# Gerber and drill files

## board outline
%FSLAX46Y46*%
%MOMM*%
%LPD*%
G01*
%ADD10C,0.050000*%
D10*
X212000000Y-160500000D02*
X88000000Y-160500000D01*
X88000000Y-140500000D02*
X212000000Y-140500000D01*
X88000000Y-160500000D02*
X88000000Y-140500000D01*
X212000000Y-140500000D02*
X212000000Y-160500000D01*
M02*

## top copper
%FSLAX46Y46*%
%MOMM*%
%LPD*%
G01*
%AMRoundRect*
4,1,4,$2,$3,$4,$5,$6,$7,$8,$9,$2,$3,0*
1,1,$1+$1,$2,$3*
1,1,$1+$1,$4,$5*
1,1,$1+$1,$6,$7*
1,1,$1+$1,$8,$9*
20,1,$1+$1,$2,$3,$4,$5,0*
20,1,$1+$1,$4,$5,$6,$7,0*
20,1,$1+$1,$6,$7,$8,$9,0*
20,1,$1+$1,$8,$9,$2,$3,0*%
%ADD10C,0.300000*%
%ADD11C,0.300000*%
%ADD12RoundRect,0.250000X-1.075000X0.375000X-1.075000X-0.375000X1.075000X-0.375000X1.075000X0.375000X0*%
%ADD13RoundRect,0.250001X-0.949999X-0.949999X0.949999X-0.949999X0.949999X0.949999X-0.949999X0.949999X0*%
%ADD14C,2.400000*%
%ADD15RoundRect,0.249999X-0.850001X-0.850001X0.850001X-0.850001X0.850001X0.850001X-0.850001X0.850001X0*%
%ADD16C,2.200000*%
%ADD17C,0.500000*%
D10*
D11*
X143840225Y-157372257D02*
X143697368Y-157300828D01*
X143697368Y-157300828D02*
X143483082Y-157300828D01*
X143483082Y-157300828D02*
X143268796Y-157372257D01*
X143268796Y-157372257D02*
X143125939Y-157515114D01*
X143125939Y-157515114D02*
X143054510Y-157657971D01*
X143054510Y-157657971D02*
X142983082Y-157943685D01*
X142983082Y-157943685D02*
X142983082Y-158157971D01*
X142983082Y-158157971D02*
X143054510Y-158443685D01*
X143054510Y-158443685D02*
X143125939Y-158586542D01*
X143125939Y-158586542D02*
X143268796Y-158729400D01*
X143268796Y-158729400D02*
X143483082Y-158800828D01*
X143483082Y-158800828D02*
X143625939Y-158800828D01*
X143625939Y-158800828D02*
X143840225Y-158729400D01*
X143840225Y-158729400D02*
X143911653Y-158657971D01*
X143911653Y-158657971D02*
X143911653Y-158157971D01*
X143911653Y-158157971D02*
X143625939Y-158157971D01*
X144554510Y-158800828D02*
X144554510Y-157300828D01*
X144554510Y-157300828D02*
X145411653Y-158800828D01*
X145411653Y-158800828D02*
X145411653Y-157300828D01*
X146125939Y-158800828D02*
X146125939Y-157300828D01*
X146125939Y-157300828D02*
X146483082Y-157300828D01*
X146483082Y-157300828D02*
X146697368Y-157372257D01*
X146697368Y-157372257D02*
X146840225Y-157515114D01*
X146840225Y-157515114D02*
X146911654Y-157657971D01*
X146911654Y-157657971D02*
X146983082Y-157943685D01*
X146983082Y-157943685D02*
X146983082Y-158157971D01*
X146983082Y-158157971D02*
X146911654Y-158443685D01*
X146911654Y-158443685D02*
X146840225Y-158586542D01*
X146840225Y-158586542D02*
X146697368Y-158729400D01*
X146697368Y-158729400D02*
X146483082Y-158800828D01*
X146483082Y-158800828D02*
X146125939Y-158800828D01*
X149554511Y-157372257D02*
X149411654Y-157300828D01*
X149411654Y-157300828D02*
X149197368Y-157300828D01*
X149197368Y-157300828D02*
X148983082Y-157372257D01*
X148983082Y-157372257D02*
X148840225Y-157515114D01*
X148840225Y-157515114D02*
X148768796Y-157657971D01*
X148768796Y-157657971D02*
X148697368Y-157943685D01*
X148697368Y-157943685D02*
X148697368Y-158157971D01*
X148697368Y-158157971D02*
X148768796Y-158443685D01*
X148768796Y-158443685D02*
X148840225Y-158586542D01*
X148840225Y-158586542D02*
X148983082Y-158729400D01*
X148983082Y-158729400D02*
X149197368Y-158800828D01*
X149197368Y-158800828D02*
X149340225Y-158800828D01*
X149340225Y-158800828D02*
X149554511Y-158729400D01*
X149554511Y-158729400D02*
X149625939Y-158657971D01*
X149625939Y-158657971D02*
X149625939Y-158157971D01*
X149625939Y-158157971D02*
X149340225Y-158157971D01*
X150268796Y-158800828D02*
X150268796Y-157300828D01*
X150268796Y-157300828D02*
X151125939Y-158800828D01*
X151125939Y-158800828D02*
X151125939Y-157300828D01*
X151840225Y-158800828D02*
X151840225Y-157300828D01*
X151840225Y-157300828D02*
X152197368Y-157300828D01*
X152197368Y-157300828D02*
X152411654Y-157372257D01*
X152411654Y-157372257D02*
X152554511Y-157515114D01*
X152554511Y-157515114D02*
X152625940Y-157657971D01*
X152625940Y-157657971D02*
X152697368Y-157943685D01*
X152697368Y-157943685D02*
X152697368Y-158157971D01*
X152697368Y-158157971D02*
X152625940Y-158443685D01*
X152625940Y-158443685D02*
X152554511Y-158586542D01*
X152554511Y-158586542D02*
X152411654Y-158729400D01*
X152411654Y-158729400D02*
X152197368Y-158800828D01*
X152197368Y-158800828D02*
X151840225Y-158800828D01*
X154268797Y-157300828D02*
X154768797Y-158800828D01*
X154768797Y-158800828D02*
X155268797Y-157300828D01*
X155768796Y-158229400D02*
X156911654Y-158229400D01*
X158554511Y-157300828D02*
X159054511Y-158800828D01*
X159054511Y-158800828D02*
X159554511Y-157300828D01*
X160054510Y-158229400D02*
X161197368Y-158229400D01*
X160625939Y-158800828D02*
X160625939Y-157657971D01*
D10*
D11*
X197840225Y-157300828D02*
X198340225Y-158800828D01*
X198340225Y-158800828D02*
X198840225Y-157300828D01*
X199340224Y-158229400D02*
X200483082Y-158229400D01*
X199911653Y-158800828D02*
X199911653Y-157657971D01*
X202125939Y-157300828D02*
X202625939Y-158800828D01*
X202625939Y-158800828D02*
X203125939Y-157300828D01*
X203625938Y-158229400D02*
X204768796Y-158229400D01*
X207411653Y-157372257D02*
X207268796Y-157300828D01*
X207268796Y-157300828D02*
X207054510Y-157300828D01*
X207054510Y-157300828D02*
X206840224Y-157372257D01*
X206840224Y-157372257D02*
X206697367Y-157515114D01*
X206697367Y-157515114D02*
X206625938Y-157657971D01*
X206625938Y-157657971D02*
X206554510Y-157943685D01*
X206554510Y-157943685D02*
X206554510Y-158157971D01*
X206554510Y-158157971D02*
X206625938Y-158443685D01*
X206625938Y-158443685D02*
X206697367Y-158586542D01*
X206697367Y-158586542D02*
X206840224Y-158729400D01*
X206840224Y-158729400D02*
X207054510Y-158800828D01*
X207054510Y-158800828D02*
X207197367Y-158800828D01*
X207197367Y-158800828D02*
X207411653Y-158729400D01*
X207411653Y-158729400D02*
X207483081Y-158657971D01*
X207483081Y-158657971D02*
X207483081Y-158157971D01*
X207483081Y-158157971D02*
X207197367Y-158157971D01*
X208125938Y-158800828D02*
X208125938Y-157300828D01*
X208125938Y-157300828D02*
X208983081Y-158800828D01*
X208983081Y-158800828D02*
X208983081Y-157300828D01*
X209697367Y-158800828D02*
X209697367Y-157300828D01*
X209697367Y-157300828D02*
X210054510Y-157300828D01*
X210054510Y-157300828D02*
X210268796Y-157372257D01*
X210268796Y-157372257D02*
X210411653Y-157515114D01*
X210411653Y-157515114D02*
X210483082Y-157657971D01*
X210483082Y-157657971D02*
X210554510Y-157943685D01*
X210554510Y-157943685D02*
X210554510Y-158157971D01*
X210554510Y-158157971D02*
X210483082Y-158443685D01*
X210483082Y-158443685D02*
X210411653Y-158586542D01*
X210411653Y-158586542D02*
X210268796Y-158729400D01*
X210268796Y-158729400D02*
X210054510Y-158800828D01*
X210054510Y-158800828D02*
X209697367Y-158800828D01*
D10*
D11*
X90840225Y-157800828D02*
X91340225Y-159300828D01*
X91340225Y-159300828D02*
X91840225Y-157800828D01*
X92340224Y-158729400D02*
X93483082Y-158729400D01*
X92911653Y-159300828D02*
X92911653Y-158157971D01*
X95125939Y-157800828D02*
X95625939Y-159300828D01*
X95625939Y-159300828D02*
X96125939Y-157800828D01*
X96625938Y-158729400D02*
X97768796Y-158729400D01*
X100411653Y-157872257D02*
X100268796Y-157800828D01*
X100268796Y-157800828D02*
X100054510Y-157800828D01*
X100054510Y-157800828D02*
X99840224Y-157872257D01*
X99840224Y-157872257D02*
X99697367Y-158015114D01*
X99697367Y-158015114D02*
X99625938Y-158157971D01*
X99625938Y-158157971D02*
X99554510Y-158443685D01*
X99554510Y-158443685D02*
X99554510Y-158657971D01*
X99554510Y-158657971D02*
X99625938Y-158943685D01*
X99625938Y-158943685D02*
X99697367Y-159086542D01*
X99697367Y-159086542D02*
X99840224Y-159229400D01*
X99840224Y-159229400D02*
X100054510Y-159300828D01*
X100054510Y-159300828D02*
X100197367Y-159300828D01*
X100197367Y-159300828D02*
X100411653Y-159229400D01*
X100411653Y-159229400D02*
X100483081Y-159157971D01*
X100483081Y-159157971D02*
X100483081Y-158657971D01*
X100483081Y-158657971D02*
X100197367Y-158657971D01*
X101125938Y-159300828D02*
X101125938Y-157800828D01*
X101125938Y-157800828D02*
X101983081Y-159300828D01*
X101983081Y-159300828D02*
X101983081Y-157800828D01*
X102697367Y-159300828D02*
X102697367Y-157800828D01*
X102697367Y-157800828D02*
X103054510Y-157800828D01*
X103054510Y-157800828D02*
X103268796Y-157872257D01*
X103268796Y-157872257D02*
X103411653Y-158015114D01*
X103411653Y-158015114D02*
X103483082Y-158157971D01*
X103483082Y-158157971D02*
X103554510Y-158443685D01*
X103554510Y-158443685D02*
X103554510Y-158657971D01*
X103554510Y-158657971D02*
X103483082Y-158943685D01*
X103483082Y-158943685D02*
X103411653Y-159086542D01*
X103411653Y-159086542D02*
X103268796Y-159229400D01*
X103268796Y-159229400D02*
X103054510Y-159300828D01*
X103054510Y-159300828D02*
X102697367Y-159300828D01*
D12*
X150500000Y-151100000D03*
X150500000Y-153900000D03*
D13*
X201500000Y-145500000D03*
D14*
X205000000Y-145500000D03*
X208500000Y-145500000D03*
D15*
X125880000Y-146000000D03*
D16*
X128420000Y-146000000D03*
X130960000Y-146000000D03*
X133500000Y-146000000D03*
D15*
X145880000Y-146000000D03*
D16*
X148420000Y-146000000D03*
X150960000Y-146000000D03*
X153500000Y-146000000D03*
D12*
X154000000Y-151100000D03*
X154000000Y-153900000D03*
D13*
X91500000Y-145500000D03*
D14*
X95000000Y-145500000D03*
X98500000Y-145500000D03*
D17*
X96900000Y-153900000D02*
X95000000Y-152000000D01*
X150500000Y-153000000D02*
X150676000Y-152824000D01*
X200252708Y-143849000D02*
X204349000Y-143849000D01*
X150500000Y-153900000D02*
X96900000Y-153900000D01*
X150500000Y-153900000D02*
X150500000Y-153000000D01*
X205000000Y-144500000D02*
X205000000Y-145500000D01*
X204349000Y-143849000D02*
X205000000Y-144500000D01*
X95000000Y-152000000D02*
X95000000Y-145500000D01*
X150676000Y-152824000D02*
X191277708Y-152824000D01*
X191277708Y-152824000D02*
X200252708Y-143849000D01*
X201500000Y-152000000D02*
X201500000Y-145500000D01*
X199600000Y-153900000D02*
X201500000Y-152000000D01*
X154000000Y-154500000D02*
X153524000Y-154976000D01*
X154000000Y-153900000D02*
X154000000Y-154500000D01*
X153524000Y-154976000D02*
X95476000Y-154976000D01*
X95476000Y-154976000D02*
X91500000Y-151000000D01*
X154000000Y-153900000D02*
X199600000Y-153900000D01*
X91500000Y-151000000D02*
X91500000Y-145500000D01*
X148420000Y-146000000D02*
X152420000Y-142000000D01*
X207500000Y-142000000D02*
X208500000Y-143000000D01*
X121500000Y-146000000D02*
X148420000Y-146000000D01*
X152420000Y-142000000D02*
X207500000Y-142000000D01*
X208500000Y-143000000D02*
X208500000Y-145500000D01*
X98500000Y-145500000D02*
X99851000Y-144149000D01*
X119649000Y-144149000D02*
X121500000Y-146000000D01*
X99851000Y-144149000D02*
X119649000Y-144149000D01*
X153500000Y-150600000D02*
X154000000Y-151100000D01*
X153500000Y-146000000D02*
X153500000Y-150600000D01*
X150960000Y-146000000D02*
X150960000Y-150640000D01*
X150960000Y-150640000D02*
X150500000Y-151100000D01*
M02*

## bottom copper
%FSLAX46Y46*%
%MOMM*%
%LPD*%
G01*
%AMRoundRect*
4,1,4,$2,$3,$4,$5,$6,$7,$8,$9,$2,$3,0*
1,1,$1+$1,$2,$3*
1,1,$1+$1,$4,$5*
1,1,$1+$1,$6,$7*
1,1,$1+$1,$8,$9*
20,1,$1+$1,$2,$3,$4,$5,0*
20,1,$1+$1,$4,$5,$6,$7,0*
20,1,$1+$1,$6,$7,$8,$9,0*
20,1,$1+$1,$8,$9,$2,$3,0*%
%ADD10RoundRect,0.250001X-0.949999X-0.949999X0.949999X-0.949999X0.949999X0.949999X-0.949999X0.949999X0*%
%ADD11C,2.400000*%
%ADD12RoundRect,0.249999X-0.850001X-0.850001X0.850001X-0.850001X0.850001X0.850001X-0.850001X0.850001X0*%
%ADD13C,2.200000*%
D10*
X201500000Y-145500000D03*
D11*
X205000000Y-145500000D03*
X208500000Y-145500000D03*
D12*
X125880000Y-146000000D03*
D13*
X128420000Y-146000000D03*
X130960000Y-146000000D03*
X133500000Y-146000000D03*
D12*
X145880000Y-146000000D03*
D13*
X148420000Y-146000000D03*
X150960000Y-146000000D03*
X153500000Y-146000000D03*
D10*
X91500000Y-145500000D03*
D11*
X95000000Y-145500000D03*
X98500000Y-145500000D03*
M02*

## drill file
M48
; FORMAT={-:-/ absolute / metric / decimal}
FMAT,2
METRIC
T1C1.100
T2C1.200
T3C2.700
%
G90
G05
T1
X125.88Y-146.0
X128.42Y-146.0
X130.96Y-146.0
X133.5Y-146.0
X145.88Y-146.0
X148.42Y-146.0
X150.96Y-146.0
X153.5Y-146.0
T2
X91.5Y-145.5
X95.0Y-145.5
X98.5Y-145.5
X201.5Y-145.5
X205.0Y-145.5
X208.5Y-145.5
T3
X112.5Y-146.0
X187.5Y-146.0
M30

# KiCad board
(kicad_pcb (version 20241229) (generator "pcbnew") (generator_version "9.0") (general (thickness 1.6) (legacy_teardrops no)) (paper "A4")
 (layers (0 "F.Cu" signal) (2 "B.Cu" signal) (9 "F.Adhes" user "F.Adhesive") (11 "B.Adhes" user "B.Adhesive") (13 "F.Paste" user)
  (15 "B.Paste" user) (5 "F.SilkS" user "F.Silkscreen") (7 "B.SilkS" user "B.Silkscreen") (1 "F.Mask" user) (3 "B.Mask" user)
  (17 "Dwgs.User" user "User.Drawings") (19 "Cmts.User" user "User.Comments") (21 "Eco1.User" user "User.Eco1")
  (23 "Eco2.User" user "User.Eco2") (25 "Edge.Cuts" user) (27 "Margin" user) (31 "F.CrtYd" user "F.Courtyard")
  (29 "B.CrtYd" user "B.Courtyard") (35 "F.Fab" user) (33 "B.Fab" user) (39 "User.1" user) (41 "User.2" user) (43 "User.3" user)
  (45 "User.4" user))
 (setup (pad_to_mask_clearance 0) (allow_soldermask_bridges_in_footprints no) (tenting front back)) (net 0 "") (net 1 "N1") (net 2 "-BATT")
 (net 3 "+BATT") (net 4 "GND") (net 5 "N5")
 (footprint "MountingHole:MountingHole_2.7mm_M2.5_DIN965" (layer "F.Cu") (at 187.5 146)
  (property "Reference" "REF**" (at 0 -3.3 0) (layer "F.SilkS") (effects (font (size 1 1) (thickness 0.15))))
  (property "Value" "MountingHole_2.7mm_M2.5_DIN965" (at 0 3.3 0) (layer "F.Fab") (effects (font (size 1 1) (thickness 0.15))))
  (pad "" np_thru_hole circle (at 0 0) (size 2.7 2.7) (drill 2.7) (layers "*.Cu" "*.Mask")))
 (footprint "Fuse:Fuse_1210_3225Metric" (layer "F.Cu") (at 150.5 152.5 -90)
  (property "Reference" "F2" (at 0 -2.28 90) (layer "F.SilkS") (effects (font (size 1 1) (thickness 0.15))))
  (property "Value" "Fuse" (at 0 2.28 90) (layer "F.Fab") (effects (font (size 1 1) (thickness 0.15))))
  (pad "1" smd roundrect (at -1.4 0 270) (size 1.25 2.65) (layers "F.Cu" "F.Mask" "F.Paste") (roundrect_rratio 0.2) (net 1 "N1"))
  (pad "2" smd roundrect (at 1.4 0 270) (size 1.25 2.65) (layers "F.Cu" "F.Mask" "F.Paste") (roundrect_rratio 0.2) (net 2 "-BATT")))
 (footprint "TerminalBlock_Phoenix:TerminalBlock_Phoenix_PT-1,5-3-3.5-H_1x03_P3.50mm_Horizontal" (layer "F.Cu") (at 201.5 145.5)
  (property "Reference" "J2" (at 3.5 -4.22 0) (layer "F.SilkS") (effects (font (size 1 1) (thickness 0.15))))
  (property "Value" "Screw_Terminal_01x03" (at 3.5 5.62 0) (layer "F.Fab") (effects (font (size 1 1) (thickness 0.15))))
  (pad "1" thru_hole roundrect (at 0 0) (size 2.4 2.4) (drill 1.2) (layers "*.Cu" "*.Mask") (remove_unused_layers no)
   (roundrect_rratio 0.104167) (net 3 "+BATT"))
  (pad "2" thru_hole circle (at 3.5 0) (size 2.4 2.4) (drill 1.2) (layers "*.Cu" "*.Mask") (remove_unused_layers no) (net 2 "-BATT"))
  (pad "3" thru_hole circle (at 7 0) (size 2.4 2.4) (drill 1.2) (layers "*.Cu" "*.Mask") (remove_unused_layers no) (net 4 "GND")))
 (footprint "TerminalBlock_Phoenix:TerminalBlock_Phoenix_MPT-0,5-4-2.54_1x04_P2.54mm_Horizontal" (layer "F.Cu") (at 125.88 146)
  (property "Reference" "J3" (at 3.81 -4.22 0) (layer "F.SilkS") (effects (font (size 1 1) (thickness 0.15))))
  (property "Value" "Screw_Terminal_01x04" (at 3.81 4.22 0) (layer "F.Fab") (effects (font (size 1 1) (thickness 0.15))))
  (pad "1" thru_hole roundrect (at 0 0) (size 2.2 2.2) (drill 1.1) (layers "*.Cu" "*.Mask") (remove_unused_layers no)
   (roundrect_rratio 0.113636) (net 4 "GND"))
  (pad "2" thru_hole circle (at 2.54 0) (size 2.2 2.2) (drill 1.1) (layers "*.Cu" "*.Mask") (remove_unused_layers no) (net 4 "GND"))
  (pad "3" thru_hole circle (at 5.08 0) (size 2.2 2.2) (drill 1.1) (layers "*.Cu" "*.Mask") (remove_unused_layers no) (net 4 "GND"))
  (pad "4" thru_hole circle (at 7.62 0) (size 2.2 2.2) (drill 1.1) (layers "*.Cu" "*.Mask") (remove_unused_layers no) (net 4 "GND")))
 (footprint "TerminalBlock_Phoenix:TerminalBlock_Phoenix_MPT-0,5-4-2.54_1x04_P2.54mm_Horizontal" (layer "F.Cu") (at 145.88 146)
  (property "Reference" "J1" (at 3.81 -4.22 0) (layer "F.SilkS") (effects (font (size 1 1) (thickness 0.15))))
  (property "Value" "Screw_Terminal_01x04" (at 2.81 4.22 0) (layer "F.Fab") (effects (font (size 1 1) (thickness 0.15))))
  (pad "1" thru_hole roundrect (at 0 0) (size 2.2 2.2) (drill 1.1) (layers "*.Cu" "*.Mask") (remove_unused_layers no)
   (roundrect_rratio 0.113636) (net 4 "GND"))
  (pad "2" thru_hole circle (at 2.54 0) (size 2.2 2.2) (drill 1.1) (layers "*.Cu" "*.Mask") (remove_unused_layers no) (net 4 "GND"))
  (pad "3" thru_hole circle (at 5.08 0) (size 2.2 2.2) (drill 1.1) (layers "*.Cu" "*.Mask") (remove_unused_layers no) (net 1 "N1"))
  (pad "4" thru_hole circle (at 7.62 0) (size 2.2 2.2) (drill 1.1) (layers "*.Cu" "*.Mask") (remove_unused_layers no) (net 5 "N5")))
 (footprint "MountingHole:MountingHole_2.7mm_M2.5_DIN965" (layer "F.Cu") (at 112.5 146)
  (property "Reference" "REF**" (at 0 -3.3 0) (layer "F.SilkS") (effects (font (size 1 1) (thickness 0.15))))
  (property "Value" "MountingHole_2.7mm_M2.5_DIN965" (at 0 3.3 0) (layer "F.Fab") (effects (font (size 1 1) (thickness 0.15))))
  (pad "" np_thru_hole circle (at 0 0) (size 2.7 2.7) (drill 2.7) (layers "*.Cu" "*.Mask")))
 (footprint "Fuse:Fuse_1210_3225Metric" (layer "F.Cu") (at 154 152.5 -90)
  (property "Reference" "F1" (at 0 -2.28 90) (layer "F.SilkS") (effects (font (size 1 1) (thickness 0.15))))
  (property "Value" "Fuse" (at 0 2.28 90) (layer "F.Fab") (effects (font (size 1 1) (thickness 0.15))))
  (pad "1" smd roundrect (at -1.4 0 270) (size 1.25 2.65) (layers "F.Cu" "F.Mask" "F.Paste") (roundrect_rratio 0.2) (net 5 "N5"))
  (pad "2" smd roundrect (at 1.4 0 270) (size 1.25 2.65) (layers "F.Cu" "F.Mask" "F.Paste") (roundrect_rratio 0.2) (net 3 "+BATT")))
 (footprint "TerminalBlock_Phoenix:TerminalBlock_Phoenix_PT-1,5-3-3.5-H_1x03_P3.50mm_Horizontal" (layer "F.Cu") (at 91.5 145.5)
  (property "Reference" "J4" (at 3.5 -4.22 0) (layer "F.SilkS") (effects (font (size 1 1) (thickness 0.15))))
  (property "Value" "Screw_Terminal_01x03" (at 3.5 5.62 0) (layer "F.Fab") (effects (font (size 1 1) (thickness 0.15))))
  (pad "1" thru_hole roundrect (at 0 0) (size 2.4 2.4) (drill 1.2) (layers "*.Cu" "*.Mask") (remove_unused_layers no)
   (roundrect_rratio 0.104167) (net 3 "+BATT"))
  (pad "2" thru_hole circle (at 3.5 0) (size 2.4 2.4) (drill 1.2) (layers "*.Cu" "*.Mask") (remove_unused_layers no) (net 2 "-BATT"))
  (pad "3" thru_hole circle (at 7 0) (size 2.4 2.4) (drill 1.2) (layers "*.Cu" "*.Mask") (remove_unused_layers no) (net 4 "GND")))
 (gr_line (start 212 160.5) (end 88 160.5) (stroke (width 0.05) (type default)) (layer "Edge.Cuts"))
 (gr_line (start 88 140.5) (end 212 140.5) (stroke (width 0.05) (type default)) (layer "Edge.Cuts"))
 (gr_line (start 88 160.5) (end 88 140.5) (stroke (width 0.05) (type default)) (layer "Edge.Cuts"))
 (gr_line (start 212 140.5) (end 212 160.5) (stroke (width 0.05) (type default)) (layer "Edge.Cuts"))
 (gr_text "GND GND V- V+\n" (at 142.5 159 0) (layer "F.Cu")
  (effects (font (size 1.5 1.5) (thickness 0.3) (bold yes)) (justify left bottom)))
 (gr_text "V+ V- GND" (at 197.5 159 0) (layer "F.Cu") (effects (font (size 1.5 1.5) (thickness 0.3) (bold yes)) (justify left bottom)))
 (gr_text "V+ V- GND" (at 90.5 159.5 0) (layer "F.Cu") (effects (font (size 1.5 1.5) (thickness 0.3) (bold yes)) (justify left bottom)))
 (segment (start 96.9 153.9) (end 95 152) (width 0.5) (layer "F.Cu") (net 2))
 (segment (start 150.5 153) (end 150.676 152.824) (width 0.5) (layer "F.Cu") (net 2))
 (segment (start 200.252708 143.849) (end 204.349 143.849) (width 0.5) (layer "F.Cu") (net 2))
 (segment (start 150.5 153.9) (end 96.9 153.9) (width 0.5) (layer "F.Cu") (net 2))
 (segment (start 150.5 153.9) (end 150.5 153) (width 0.5) (layer "F.Cu") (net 2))
 (segment (start 205 144.5) (end 205 145.5) (width 0.5) (layer "F.Cu") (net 2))
 (segment (start 204.349 143.849) (end 205 144.5) (width 0.5) (layer "F.Cu") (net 2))
 (segment (start 95 152) (end 95 145.5) (width 0.5) (layer "F.Cu") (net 2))
 (segment (start 150.676 152.824) (end 191.277708 152.824) (width 0.5) (layer "F.Cu") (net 2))
 (segment (start 191.277708 152.824) (end 200.252708 143.849) (width 0.5) (layer "F.Cu") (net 2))
 (segment (start 201.5 152) (end 201.5 145.5) (width 0.5) (layer "F.Cu") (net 3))
 (segment (start 199.6 153.9) (end 201.5 152) (width 0.5) (layer "F.Cu") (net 3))
 (segment (start 154 154.5) (end 153.524 154.976) (width 0.5) (layer "F.Cu") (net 3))
 (segment (start 154 153.9) (end 154 154.5) (width 0.5) (layer "F.Cu") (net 3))
 (segment (start 153.524 154.976) (end 95.476 154.976) (width 0.5) (layer "F.Cu") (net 3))
 (segment (start 95.476 154.976) (end 91.5 151) (width 0.5) (layer "F.Cu") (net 3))
 (segment (start 154 153.9) (end 199.6 153.9) (width 0.5) (layer "F.Cu") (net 3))
 (segment (start 91.5 151) (end 91.5 145.5) (width 0.5) (layer "F.Cu") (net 3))
 (segment (start 148.42 146) (end 152.42 142) (width 0.5) (layer "F.Cu") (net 4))
 (segment (start 207.5 142) (end 208.5 143) (width 0.5) (layer "F.Cu") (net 4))
 (segment (start 121.5 146) (end 148.42 146) (width 0.5) (layer "F.Cu") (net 4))
 (segment (start 152.42 142) (end 207.5 142) (width 0.5) (layer "F.Cu") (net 4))
 (segment (start 208.5 143) (end 208.5 145.5) (width 0.5) (layer "F.Cu") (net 4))
 (segment (start 98.5 145.5) (end 99.851 144.149) (width 0.5) (layer "F.Cu") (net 4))
 (segment (start 119.649 144.149) (end 121.5 146) (width 0.5) (layer "F.Cu") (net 4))
 (segment (start 99.851 144.149) (end 119.649 144.149) (width 0.5) (layer "F.Cu") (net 4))
 (segment (start 153.5 150.6) (end 154 151.1) (width 0.5) (layer "F.Cu") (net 5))
 (segment (start 153.5 146) (end 153.5 150.6) (width 0.5) (layer "F.Cu") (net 5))
 (segment (start 150.96 146) (end 150.96 150.64) (width 0.5) (layer "F.Cu") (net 1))
 (segment (start 150.96 150.64) (end 150.5 151.1) (width 0.5) (layer "F.Cu") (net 1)))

